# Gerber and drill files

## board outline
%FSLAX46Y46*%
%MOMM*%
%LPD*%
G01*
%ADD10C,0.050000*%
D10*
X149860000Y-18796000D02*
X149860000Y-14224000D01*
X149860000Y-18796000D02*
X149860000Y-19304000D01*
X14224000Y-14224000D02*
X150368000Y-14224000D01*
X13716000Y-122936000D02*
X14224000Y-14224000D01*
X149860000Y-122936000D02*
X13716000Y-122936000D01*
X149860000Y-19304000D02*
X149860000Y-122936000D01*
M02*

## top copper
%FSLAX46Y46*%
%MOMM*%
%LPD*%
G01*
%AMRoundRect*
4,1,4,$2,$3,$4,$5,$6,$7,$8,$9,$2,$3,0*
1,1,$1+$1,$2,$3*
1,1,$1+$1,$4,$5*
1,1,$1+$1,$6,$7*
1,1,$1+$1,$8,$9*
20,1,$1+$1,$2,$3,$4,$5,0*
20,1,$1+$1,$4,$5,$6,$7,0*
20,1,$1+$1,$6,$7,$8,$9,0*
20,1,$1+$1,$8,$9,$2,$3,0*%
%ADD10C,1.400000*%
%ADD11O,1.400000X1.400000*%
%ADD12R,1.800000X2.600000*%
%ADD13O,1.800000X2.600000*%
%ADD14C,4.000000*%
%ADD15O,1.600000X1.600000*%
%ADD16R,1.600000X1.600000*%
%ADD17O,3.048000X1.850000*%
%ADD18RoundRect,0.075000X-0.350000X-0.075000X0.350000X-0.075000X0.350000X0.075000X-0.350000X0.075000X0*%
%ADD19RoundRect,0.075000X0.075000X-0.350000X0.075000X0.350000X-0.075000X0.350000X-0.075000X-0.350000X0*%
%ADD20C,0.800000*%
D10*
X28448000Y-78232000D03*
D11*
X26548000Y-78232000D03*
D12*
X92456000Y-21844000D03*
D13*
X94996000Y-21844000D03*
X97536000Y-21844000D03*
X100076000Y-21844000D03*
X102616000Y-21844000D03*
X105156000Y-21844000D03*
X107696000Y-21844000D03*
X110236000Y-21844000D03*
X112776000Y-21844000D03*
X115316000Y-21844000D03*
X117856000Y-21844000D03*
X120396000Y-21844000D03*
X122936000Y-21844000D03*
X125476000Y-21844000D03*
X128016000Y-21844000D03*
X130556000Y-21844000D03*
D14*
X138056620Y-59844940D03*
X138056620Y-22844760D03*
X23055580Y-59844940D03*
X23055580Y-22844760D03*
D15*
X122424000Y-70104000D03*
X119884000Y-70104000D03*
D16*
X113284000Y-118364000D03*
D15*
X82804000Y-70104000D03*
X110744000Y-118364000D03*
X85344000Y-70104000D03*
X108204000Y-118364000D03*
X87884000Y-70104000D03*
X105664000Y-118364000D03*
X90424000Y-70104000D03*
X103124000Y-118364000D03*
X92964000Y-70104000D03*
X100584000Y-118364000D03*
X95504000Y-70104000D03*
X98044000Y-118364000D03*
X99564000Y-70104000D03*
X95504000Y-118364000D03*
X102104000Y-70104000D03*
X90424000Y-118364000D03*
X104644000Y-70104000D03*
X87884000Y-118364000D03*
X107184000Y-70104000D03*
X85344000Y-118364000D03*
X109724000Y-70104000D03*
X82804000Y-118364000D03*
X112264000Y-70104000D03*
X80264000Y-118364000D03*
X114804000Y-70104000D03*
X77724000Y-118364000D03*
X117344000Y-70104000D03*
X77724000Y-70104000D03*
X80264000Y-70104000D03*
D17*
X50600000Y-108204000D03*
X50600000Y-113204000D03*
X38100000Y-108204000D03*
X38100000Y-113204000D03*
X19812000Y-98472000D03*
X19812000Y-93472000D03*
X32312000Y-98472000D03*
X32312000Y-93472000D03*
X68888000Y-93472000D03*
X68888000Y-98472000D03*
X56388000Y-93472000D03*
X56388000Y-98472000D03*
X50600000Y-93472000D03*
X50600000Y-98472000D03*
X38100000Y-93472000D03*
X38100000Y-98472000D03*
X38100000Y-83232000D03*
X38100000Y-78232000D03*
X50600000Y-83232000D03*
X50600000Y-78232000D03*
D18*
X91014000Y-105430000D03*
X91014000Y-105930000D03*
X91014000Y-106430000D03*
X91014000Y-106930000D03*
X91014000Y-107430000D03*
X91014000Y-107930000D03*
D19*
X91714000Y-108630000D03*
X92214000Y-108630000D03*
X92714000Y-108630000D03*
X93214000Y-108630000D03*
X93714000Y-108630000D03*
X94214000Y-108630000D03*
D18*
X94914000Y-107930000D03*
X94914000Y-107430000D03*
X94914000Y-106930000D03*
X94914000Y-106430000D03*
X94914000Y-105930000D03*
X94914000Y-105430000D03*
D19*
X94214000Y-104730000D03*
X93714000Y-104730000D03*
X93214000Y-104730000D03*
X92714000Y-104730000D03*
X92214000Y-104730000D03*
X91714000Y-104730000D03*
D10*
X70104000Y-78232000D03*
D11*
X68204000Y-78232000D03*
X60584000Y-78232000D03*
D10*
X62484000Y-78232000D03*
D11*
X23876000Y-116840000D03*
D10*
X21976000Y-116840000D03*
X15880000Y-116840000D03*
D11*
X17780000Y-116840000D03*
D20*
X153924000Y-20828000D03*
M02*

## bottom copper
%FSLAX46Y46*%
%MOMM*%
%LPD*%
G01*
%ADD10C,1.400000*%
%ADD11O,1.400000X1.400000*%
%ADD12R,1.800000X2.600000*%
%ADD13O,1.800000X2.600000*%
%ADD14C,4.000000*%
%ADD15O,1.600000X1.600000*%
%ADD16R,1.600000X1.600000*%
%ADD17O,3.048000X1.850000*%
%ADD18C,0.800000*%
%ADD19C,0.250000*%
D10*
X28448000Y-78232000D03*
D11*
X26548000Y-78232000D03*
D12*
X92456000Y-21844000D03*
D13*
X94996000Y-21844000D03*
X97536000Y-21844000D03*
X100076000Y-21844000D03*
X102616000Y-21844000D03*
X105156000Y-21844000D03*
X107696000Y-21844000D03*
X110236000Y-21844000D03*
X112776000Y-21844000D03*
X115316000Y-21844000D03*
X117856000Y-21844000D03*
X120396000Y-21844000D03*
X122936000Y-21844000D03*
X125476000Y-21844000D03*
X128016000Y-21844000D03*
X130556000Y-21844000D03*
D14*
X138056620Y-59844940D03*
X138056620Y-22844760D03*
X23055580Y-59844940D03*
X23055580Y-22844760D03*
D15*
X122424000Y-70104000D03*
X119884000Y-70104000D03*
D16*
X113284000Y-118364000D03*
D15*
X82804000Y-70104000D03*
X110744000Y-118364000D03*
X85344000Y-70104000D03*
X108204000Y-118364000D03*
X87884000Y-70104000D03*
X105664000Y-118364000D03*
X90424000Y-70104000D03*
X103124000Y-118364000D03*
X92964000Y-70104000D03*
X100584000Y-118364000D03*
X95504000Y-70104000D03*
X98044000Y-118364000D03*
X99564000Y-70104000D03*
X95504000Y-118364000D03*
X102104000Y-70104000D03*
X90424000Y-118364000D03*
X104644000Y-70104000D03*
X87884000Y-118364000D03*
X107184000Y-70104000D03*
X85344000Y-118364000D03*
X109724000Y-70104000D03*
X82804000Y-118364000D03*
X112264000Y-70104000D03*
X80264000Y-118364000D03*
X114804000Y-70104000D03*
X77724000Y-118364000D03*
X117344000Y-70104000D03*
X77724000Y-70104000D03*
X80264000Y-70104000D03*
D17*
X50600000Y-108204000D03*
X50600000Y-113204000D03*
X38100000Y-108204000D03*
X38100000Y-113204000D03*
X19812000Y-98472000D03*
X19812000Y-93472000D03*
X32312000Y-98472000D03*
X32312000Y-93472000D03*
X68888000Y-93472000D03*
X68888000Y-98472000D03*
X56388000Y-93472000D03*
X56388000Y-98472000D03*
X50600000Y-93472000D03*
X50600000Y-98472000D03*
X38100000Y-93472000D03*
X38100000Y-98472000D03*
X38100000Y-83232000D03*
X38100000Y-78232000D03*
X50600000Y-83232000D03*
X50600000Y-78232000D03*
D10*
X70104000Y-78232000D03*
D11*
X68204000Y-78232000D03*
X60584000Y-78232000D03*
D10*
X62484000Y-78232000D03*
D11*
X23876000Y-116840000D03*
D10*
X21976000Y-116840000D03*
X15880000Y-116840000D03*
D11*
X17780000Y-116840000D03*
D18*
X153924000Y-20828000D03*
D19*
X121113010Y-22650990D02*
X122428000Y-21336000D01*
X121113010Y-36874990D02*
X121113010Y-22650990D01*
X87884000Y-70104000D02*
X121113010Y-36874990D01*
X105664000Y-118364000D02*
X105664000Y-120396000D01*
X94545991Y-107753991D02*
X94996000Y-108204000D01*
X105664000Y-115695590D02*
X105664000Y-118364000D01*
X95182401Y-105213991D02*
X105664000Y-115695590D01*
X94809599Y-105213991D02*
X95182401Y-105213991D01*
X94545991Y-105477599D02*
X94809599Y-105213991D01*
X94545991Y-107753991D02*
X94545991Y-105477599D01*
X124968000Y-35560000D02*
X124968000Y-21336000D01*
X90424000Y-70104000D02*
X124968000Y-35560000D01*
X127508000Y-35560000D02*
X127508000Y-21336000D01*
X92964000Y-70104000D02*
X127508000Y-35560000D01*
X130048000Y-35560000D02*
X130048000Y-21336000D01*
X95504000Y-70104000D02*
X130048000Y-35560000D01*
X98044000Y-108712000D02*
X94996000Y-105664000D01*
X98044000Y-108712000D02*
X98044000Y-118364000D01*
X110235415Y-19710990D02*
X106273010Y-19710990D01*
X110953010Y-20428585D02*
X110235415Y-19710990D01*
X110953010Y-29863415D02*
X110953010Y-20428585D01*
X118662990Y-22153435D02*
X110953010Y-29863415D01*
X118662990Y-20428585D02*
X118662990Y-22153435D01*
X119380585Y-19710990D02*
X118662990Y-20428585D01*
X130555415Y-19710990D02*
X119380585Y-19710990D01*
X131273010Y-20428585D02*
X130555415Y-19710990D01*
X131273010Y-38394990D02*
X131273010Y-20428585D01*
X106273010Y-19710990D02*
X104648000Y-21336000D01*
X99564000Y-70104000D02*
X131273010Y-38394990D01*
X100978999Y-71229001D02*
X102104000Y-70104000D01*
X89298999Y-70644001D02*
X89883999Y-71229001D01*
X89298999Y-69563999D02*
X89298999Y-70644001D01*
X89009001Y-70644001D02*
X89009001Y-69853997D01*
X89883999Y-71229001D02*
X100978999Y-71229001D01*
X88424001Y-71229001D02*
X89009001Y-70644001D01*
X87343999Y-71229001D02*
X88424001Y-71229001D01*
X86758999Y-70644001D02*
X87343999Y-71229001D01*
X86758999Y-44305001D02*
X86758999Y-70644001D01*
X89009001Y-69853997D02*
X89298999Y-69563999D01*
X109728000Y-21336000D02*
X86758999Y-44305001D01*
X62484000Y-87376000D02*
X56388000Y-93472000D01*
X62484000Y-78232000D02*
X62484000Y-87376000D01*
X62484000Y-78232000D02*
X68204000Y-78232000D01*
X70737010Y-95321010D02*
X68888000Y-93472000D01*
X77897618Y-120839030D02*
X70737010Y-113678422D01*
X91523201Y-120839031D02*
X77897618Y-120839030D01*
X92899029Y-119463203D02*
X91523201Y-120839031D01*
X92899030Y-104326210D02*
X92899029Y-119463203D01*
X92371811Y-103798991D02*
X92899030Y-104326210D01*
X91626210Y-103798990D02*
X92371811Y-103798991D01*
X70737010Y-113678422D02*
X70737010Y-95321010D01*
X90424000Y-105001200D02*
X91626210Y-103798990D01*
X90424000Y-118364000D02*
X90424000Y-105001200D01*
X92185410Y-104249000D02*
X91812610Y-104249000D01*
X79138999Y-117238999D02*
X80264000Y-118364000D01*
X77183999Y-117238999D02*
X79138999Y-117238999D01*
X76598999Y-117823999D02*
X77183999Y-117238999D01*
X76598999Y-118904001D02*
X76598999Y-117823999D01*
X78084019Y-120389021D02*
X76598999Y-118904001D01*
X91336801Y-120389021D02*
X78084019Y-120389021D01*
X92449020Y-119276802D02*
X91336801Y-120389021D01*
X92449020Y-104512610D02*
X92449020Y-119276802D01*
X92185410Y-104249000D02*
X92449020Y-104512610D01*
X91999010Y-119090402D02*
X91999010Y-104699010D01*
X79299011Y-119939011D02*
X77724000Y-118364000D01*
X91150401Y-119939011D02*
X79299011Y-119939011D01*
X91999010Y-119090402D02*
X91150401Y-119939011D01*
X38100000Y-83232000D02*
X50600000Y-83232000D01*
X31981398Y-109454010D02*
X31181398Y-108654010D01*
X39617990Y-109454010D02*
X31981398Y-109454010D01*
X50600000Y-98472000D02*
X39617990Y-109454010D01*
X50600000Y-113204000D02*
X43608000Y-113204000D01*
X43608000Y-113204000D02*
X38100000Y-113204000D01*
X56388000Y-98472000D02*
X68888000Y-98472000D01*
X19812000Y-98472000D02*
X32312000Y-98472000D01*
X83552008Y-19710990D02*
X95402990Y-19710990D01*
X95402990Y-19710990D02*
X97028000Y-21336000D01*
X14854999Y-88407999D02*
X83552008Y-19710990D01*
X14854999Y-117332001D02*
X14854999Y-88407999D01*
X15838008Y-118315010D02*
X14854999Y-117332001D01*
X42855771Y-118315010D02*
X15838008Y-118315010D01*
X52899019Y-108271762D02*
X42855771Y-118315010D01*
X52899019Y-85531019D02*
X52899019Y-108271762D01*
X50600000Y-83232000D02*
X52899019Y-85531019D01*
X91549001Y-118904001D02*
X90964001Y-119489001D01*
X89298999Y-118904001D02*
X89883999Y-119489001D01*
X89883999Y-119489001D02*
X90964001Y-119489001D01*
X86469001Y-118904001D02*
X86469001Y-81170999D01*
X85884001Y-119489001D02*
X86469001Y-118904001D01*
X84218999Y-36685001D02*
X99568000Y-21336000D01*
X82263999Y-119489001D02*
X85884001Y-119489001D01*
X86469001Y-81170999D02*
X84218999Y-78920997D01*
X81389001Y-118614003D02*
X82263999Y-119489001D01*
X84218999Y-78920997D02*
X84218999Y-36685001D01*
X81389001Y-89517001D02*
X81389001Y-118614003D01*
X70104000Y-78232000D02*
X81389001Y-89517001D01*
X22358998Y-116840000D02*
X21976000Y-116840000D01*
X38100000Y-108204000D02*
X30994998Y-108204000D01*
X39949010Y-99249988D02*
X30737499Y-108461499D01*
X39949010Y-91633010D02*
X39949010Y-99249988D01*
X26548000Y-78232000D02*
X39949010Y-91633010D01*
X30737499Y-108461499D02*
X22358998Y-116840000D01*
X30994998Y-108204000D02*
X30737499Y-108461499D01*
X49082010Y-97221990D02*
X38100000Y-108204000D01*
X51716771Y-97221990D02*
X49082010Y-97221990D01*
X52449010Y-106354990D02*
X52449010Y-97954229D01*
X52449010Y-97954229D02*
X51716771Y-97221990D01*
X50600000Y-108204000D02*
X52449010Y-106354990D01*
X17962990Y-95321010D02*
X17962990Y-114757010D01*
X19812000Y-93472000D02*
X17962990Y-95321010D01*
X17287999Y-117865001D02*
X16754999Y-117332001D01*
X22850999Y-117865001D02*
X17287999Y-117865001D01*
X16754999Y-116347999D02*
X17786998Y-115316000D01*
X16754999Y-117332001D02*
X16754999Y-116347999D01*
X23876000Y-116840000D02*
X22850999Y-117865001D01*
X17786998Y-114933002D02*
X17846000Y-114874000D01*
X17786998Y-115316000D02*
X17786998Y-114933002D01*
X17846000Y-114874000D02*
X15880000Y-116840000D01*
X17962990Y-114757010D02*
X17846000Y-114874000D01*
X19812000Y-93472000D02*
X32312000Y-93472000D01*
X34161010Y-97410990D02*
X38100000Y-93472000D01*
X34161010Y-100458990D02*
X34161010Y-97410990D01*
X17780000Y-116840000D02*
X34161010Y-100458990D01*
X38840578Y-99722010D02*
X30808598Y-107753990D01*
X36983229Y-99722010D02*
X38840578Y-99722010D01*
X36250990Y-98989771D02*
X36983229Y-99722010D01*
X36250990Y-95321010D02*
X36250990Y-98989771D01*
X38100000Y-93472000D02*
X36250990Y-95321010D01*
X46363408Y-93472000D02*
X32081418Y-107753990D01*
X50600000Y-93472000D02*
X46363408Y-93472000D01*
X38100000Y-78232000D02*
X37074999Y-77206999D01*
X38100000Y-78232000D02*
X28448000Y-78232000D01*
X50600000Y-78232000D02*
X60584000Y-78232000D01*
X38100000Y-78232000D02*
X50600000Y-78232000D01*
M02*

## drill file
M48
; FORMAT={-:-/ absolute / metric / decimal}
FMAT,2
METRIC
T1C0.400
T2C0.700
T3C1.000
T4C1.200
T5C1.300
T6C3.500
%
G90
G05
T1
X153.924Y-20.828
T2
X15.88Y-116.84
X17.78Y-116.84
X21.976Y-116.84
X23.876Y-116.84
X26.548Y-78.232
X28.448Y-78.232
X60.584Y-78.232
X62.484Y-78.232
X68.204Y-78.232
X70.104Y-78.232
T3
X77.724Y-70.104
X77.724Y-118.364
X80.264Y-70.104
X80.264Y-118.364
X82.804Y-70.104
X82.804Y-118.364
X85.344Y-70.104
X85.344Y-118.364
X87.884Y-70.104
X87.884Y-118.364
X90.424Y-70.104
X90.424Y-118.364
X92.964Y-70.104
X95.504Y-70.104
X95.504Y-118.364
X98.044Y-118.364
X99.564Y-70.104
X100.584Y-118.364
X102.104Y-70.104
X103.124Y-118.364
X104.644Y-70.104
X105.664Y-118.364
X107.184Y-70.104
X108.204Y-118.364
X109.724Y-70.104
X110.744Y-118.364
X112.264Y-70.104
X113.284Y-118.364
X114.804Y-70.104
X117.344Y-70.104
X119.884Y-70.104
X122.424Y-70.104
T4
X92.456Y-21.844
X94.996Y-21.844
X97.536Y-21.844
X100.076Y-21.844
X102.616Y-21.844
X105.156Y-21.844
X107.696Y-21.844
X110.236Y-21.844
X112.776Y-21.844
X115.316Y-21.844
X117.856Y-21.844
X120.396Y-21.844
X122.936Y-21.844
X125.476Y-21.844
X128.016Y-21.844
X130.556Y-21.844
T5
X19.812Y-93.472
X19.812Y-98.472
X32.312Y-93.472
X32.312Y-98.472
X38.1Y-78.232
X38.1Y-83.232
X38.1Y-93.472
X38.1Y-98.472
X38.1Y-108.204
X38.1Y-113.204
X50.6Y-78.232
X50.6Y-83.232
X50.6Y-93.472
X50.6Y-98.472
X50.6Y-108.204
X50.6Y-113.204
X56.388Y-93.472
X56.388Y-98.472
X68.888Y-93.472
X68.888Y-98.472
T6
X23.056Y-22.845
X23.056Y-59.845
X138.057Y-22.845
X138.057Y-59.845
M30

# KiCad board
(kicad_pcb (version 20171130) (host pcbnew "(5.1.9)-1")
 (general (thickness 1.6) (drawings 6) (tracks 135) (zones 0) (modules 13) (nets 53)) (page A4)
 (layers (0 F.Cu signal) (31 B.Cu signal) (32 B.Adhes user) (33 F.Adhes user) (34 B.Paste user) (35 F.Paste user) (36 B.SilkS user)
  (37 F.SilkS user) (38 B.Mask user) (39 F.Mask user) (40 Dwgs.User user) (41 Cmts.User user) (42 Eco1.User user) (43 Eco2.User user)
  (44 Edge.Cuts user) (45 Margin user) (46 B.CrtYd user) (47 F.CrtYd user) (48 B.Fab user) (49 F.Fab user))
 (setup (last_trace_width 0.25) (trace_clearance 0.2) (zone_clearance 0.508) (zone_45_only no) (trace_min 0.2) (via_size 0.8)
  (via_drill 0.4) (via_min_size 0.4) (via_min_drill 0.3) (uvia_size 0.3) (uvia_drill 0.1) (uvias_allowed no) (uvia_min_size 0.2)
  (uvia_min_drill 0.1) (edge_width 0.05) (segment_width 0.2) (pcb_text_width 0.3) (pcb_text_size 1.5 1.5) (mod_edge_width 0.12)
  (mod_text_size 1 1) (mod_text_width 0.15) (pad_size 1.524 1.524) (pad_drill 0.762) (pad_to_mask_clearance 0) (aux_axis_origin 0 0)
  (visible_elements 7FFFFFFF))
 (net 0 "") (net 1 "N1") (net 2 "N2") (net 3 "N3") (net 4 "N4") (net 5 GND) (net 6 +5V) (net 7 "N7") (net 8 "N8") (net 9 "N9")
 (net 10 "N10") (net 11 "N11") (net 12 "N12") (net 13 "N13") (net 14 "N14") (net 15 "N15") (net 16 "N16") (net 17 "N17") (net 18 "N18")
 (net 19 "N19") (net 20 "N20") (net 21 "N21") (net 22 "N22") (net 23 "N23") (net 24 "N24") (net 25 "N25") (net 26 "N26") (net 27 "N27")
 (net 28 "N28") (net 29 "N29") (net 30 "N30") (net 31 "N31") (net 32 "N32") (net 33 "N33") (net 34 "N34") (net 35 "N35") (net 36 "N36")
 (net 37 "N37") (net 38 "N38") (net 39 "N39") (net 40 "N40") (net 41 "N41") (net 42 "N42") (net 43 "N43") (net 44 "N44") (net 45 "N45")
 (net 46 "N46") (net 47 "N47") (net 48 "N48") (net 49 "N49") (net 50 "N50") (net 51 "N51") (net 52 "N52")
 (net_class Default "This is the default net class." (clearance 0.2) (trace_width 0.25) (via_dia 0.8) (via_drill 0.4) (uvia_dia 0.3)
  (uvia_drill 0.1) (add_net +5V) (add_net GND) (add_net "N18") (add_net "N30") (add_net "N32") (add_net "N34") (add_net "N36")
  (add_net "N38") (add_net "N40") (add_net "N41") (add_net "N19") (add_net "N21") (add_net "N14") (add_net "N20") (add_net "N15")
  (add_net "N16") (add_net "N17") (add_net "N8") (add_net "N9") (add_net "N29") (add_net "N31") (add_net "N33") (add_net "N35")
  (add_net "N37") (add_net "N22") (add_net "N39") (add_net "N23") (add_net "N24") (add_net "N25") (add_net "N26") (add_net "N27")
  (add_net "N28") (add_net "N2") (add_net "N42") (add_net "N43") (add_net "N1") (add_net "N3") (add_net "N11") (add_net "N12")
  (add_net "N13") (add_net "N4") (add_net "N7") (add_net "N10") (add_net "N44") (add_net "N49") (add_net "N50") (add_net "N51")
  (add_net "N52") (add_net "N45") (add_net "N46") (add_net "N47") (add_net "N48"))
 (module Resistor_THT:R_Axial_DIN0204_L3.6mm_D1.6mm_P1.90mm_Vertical (layer F.Cu) (at 28.448 78.232 180)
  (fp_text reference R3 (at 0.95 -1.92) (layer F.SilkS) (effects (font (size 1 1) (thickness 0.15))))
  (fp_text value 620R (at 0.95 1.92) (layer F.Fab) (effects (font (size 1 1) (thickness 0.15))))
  (pad 1 thru_hole circle (at 0 0 180) (size 1.4 1.4) (drill 0.7) (layers *.Cu *.Mask) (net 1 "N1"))
  (pad 2 thru_hole oval (at 1.9 0 180) (size 1.4 1.4) (drill 0.7) (layers *.Cu *.Mask) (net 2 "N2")))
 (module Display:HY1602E (layer F.Cu) (at 92.456 21.844)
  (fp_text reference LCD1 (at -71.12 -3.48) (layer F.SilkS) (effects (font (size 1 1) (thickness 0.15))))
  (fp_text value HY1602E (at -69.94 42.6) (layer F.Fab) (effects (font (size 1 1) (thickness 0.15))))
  (pad 1 thru_hole rect (at 0 0 180) (size 1.8 2.6) (drill 1.2) (layers *.Cu *.Mask) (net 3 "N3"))
  (pad 2 thru_hole oval (at 2.54 0 180) (size 1.8 2.6) (drill 1.2) (layers *.Cu *.Mask) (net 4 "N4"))
  (pad 3 thru_hole oval (at 5.08 0 180) (size 1.8 2.6) (drill 1.2) (layers *.Cu *.Mask) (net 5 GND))
  (pad 4 thru_hole oval (at 7.62 0 180) (size 1.8 2.6) (drill 1.2) (layers *.Cu *.Mask) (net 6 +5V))
  (pad 5 thru_hole oval (at 10.16 0 180) (size 1.8 2.6) (drill 1.2) (layers *.Cu *.Mask) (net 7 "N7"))
  (pad 6 thru_hole oval (at 12.7 0 180) (size 1.8 2.6) (drill 1.2) (layers *.Cu *.Mask) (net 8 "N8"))
  (pad 7 thru_hole oval (at 15.24 0 180) (size 1.8 2.6) (drill 1.2) (layers *.Cu *.Mask) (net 5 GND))
  (pad 8 thru_hole oval (at 17.78 0 180) (size 1.8 2.6) (drill 1.2) (layers *.Cu *.Mask) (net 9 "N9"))
  (pad 9 thru_hole oval (at 20.32 0 180) (size 1.8 2.6) (drill 1.2) (layers *.Cu *.Mask) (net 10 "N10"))
  (pad 10 thru_hole oval (at 22.86 0 180) (size 1.8 2.6) (drill 1.2) (layers *.Cu *.Mask) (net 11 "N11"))
  (pad 11 thru_hole oval (at 25.4 0 180) (size 1.8 2.6) (drill 1.2) (layers *.Cu *.Mask) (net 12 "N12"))
  (pad 12 thru_hole oval (at 27.94 0 180) (size 1.8 2.6) (drill 1.2) (layers *.Cu *.Mask) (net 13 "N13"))
  (pad 13 thru_hole oval (at 30.48 0 180) (size 1.8 2.6) (drill 1.2) (layers *.Cu *.Mask) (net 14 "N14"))
  (pad 14 thru_hole oval (at 33.02 0 180) (size 1.8 2.6) (drill 1.2) (layers *.Cu *.Mask) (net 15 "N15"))
  (pad 15 thru_hole oval (at 35.56 0 180) (size 1.8 2.6) (drill 1.2) (layers *.Cu *.Mask) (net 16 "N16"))
  (pad 16 thru_hole oval (at 38.1 0 180) (size 1.8 2.6) (drill 1.2) (layers *.Cu *.Mask) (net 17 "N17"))
  (pad "" thru_hole circle (at 45.60062 38.00094 180) (size 4 4) (drill 3.5) (layers *.Cu *.Mask))
  (pad "" thru_hole circle (at 45.60062 1.00076 180) (size 4 4) (drill 3.5) (layers *.Cu *.Mask))
  (pad "" thru_hole circle (at -69.40042 38.00094 180) (size 4 4) (drill 3.5) (layers *.Cu *.Mask))
  (pad "" thru_hole circle (at -69.40042 1.00076 180) (size 4 4) (drill 3.5) (layers *.Cu *.Mask)))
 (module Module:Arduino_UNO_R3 (layer F.Cu) (at 113.284 118.364 180)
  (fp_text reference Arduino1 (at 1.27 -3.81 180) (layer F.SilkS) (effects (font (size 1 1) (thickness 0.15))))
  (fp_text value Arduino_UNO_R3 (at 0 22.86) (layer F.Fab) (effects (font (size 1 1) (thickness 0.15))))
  (pad 32 thru_hole oval (at -9.14 48.26 270) (size 1.6 1.6) (drill 1) (layers *.Cu *.Mask))
  (pad 31 thru_hole oval (at -6.6 48.26 270) (size 1.6 1.6) (drill 1) (layers *.Cu *.Mask))
  (pad 1 thru_hole rect (at 0 0 270) (size 1.6 1.6) (drill 1) (layers *.Cu *.Mask) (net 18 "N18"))
  (pad 17 thru_hole oval (at 30.48 48.26 270) (size 1.6 1.6) (drill 1) (layers *.Cu *.Mask) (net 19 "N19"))
  (pad 2 thru_hole oval (at 2.54 0 270) (size 1.6 1.6) (drill 1) (layers *.Cu *.Mask) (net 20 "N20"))
  (pad 18 thru_hole oval (at 27.94 48.26 270) (size 1.6 1.6) (drill 1) (layers *.Cu *.Mask) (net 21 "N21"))
  (pad 3 thru_hole oval (at 5.08 0 270) (size 1.6 1.6) (drill 1) (layers *.Cu *.Mask) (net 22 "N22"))
  (pad 19 thru_hole oval (at 25.4 48.26 270) (size 1.6 1.6) (drill 1) (layers *.Cu *.Mask) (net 14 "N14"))
  (pad 4 thru_hole oval (at 7.62 0 270) (size 1.6 1.6) (drill 1) (layers *.Cu *.Mask) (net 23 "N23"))
  (pad 20 thru_hole oval (at 22.86 48.26 270) (size 1.6 1.6) (drill 1) (layers *.Cu *.Mask) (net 15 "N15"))
  (pad 5 thru_hole oval (at 10.16 0 270) (size 1.6 1.6) (drill 1) (layers *.Cu *.Mask) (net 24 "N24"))
  (pad 21 thru_hole oval (at 20.32 48.26 270) (size 1.6 1.6) (drill 1) (layers *.Cu *.Mask) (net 16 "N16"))
  (pad 6 thru_hole oval (at 12.7 0 270) (size 1.6 1.6) (drill 1) (layers *.Cu *.Mask) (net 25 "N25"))
  (pad 22 thru_hole oval (at 17.78 48.26 270) (size 1.6 1.6) (drill 1) (layers *.Cu *.Mask) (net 17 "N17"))
  (pad 7 thru_hole oval (at 15.24 0 270) (size 1.6 1.6) (drill 1) (layers *.Cu *.Mask) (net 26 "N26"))
  (pad 23 thru_hole oval (at 13.72 48.26 270) (size 1.6 1.6) (drill 1) (layers *.Cu *.Mask) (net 8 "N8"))
  (pad 8 thru_hole oval (at 17.78 0 270) (size 1.6 1.6) (drill 1) (layers *.Cu *.Mask) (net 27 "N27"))
  (pad 24 thru_hole oval (at 11.18 48.26 270) (size 1.6 1.6) (drill 1) (layers *.Cu *.Mask) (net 9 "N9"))
  (pad 9 thru_hole oval (at 22.86 0 270) (size 1.6 1.6) (drill 1) (layers *.Cu *.Mask) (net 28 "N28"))
  (pad 25 thru_hole oval (at 8.64 48.26 270) (size 1.6 1.6) (drill 1) (layers *.Cu *.Mask) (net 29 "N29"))
  (pad 10 thru_hole oval (at 25.4 0 270) (size 1.6 1.6) (drill 1) (layers *.Cu *.Mask) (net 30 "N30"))
  (pad 26 thru_hole oval (at 6.1 48.26 270) (size 1.6 1.6) (drill 1) (layers *.Cu *.Mask) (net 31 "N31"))
  (pad 11 thru_hole oval (at 27.94 0 270) (size 1.6 1.6) (drill 1) (layers *.Cu *.Mask) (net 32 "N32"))
  (pad 27 thru_hole oval (at 3.56 48.26 270) (size 1.6 1.6) (drill 1) (layers *.Cu *.Mask) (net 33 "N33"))
  (pad 12 thru_hole oval (at 30.48 0 270) (size 1.6 1.6) (drill 1) (layers *.Cu *.Mask) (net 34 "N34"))
  (pad 28 thru_hole oval (at 1.02 48.26 270) (size 1.6 1.6) (drill 1) (layers *.Cu *.Mask) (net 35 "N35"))
  (pad 13 thru_hole oval (at 33.02 0 270) (size 1.6 1.6) (drill 1) (layers *.Cu *.Mask) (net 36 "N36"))
  (pad 29 thru_hole oval (at -1.52 48.26 270) (size 1.6 1.6) (drill 1) (layers *.Cu *.Mask) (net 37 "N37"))
  (pad 14 thru_hole oval (at 35.56 0 270) (size 1.6 1.6) (drill 1) (layers *.Cu *.Mask) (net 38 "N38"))
  (pad 30 thru_hole oval (at -4.06 48.26 270) (size 1.6 1.6) (drill 1) (layers *.Cu *.Mask) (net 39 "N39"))
  (pad 15 thru_hole oval (at 35.56 48.26 270) (size 1.6 1.6) (drill 1) (layers *.Cu *.Mask) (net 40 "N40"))
  (pad 16 thru_hole oval (at 33.02 48.26 270) (size 1.6 1.6) (drill 1) (layers *.Cu *.Mask) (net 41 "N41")))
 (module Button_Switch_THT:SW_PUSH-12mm (layer F.Cu) (at 38.1 108.204)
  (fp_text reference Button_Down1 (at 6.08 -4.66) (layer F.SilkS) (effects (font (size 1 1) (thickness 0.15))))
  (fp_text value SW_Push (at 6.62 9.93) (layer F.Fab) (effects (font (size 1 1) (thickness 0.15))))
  (pad 1 thru_hole oval (at 12.5 0) (size 3.048 1.85) (drill 1.3) (layers *.Cu *.Mask) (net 2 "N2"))
  (pad 2 thru_hole oval (at 12.5 5) (size 3.048 1.85) (drill 1.3) (layers *.Cu *.Mask) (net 5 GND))
  (pad 1 thru_hole oval (at 0 0) (size 3.048 1.85) (drill 1.3) (layers *.Cu *.Mask) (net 2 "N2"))
  (pad 2 thru_hole oval (at 0 5) (size 3.048 1.85) (drill 1.3) (layers *.Cu *.Mask) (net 5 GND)))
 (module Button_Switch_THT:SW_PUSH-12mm (layer F.Cu) (at 19.812 93.472)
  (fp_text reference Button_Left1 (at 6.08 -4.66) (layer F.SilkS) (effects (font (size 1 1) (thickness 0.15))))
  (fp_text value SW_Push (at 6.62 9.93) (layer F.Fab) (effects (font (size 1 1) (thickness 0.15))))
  (pad 2 thru_hole oval (at 0 5) (size 3.048 1.85) (drill 1.3) (layers *.Cu *.Mask) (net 5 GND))
  (pad 1 thru_hole oval (at 0 0) (size 3.048 1.85) (drill 1.3) (layers *.Cu *.Mask) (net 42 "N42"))
  (pad 2 thru_hole oval (at 12.5 5) (size 3.048 1.85) (drill 1.3) (layers *.Cu *.Mask) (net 5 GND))
  (pad 1 thru_hole oval (at 12.5 0) (size 3.048 1.85) (drill 1.3) (layers *.Cu *.Mask) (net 42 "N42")))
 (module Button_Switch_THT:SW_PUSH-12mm (layer F.Cu) (at 56.388 93.472)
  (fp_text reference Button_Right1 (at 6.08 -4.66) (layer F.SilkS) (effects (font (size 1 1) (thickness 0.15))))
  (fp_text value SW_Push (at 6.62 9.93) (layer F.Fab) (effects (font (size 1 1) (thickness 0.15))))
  (pad 1 thru_hole oval (at 12.5 0) (size 3.048 1.85) (drill 1.3) (layers *.Cu *.Mask) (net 28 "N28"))
  (pad 2 thru_hole oval (at 12.5 5) (size 3.048 1.85) (drill 1.3) (layers *.Cu *.Mask) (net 5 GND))
  (pad 1 thru_hole oval (at 0 0) (size 3.048 1.85) (drill 1.3) (layers *.Cu *.Mask) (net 28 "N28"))
  (pad 2 thru_hole oval (at 0 5) (size 3.048 1.85) (drill 1.3) (layers *.Cu *.Mask) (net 5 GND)))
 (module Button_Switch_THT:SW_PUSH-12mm (layer F.Cu) (at 38.1 93.472)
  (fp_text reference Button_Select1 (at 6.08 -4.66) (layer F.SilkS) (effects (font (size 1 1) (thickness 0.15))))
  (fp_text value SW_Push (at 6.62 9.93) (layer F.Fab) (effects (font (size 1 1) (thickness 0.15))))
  (pad 1 thru_hole oval (at 12.5 0) (size 3.048 1.85) (drill 1.3) (layers *.Cu *.Mask) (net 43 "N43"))
  (pad 2 thru_hole oval (at 12.5 5) (size 3.048 1.85) (drill 1.3) (layers *.Cu *.Mask) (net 5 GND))
  (pad 1 thru_hole oval (at 0 0) (size 3.048 1.85) (drill 1.3) (layers *.Cu *.Mask) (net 43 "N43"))
  (pad 2 thru_hole oval (at 0 5) (size 3.048 1.85) (drill 1.3) (layers *.Cu *.Mask) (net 5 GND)))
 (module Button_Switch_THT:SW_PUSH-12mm (layer F.Cu) (at 38.1 78.232)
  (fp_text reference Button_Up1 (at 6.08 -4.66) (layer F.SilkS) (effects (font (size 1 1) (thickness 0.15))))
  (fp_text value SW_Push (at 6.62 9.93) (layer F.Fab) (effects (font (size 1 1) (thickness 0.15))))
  (pad 2 thru_hole oval (at 0 5) (size 3.048 1.85) (drill 1.3) (layers *.Cu *.Mask) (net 5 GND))
  (pad 1 thru_hole oval (at 0 0) (size 3.048 1.85) (drill 1.3) (layers *.Cu *.Mask) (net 1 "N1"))
  (pad 2 thru_hole oval (at 12.5 5) (size 3.048 1.85) (drill 1.3) (layers *.Cu *.Mask) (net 5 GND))
  (pad 1 thru_hole oval (at 12.5 0) (size 3.048 1.85) (drill 1.3) (layers *.Cu *.Mask) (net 1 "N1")))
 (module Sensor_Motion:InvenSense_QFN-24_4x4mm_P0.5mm (layer F.Cu) (at 92.964 106.68)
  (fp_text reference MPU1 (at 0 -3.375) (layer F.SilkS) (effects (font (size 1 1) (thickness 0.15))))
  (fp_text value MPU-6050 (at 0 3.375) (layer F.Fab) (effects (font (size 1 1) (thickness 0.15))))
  (pad 1 smd roundrect (at -1.95 -1.25) (size 0.85 0.3) (layers F.Cu F.Paste F.Mask) (roundrect_rratio 0.25) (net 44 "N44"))
  (pad 2 smd roundrect (at -1.95 -0.75) (size 0.85 0.3) (layers F.Cu F.Paste F.Mask) (roundrect_rratio 0.25))
  (pad 3 smd roundrect (at -1.95 -0.25) (size 0.85 0.3) (layers F.Cu F.Paste F.Mask) (roundrect_rratio 0.25))
  (pad 4 smd roundrect (at -1.95 0.25) (size 0.85 0.3) (layers F.Cu F.Paste F.Mask) (roundrect_rratio 0.25))
  (pad 5 smd roundrect (at -1.95 0.75) (size 0.85 0.3) (layers F.Cu F.Paste F.Mask) (roundrect_rratio 0.25))
  (pad 6 smd roundrect (at -1.95 1.25) (size 0.85 0.3) (layers F.Cu F.Paste F.Mask) (roundrect_rratio 0.25) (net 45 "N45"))
  (pad 7 smd roundrect (at -1.25 1.95 90) (size 0.85 0.3) (layers F.Cu F.Paste F.Mask) (roundrect_rratio 0.25) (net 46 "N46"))
  (pad 8 smd roundrect (at -0.75 1.95 90) (size 0.85 0.3) (layers F.Cu F.Paste F.Mask) (roundrect_rratio 0.25) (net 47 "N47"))
  (pad 9 smd roundrect (at -0.25 1.95 90) (size 0.85 0.3) (layers F.Cu F.Paste F.Mask) (roundrect_rratio 0.25) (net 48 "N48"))
  (pad 10 smd roundrect (at 0.25 1.95 90) (size 0.85 0.3) (layers F.Cu F.Paste F.Mask) (roundrect_rratio 0.25) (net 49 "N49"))
  (pad 11 smd roundrect (at 0.75 1.95 90) (size 0.85 0.3) (layers F.Cu F.Paste F.Mask) (roundrect_rratio 0.25) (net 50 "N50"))
  (pad 12 smd roundrect (at 1.25 1.95 90) (size 0.85 0.3) (layers F.Cu F.Paste F.Mask) (roundrect_rratio 0.25) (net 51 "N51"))
  (pad 13 smd roundrect (at 1.95 1.25) (size 0.85 0.3) (layers F.Cu F.Paste F.Mask) (roundrect_rratio 0.25) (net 23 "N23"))
  (pad 14 smd roundrect (at 1.95 0.75) (size 0.85 0.3) (layers F.Cu F.Paste F.Mask) (roundrect_rratio 0.25))
  (pad 15 smd roundrect (at 1.95 0.25) (size 0.85 0.3) (layers F.Cu F.Paste F.Mask) (roundrect_rratio 0.25))
  (pad 16 smd roundrect (at 1.95 -0.25) (size 0.85 0.3) (layers F.Cu F.Paste F.Mask) (roundrect_rratio 0.25))
  (pad 17 smd roundrect (at 1.95 -0.75) (size 0.85 0.3) (layers F.Cu F.Paste F.Mask) (roundrect_rratio 0.25))
  (pad 18 smd roundrect (at 1.95 -1.25) (size 0.85 0.3) (layers F.Cu F.Paste F.Mask) (roundrect_rratio 0.25) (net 26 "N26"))
  (pad 19 smd roundrect (at 1.25 -1.95 90) (size 0.85 0.3) (layers F.Cu F.Paste F.Mask) (roundrect_rratio 0.25))
  (pad 20 smd roundrect (at 0.75 -1.95 90) (size 0.85 0.3) (layers F.Cu F.Paste F.Mask) (roundrect_rratio 0.25) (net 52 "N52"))
  (pad 21 smd roundrect (at 0.25 -1.95 90) (size 0.85 0.3) (layers F.Cu F.Paste F.Mask) (roundrect_rratio 0.25))
  (pad 22 smd roundrect (at -0.25 -1.95 90) (size 0.85 0.3) (layers F.Cu F.Paste F.Mask) (roundrect_rratio 0.25))
  (pad 23 smd roundrect (at -0.75 -1.95 90) (size 0.85 0.3) (layers F.Cu F.Paste F.Mask) (roundrect_rratio 0.25) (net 38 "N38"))
  (pad 24 smd roundrect (at -1.25 -1.95 90) (size 0.85 0.3) (layers F.Cu F.Paste F.Mask) (roundrect_rratio 0.25) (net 36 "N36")))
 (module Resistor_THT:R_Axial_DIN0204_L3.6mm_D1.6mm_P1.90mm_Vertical (layer F.Cu) (at 70.104 78.232 180)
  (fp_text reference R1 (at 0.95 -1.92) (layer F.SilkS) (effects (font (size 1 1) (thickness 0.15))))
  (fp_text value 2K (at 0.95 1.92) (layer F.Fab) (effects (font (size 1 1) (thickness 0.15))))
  (pad 1 thru_hole circle (at 0 0 180) (size 1.4 1.4) (drill 0.7) (layers *.Cu *.Mask) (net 6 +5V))
  (pad 2 thru_hole oval (at 1.9 0 180) (size 1.4 1.4) (drill 0.7) (layers *.Cu *.Mask) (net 28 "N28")))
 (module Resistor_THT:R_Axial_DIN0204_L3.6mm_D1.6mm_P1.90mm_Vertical (layer F.Cu) (at 62.484 78.232 180)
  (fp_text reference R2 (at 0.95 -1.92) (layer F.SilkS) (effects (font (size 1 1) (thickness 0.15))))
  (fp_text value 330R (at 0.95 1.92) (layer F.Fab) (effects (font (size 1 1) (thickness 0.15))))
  (pad 2 thru_hole oval (at 1.9 0 180) (size 1.4 1.4) (drill 0.7) (layers *.Cu *.Mask) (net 1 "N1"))
  (pad 1 thru_hole circle (at 0 0 180) (size 1.4 1.4) (drill 0.7) (layers *.Cu *.Mask) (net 28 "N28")))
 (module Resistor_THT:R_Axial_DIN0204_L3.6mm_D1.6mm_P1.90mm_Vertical (layer F.Cu) (at 21.976 116.84)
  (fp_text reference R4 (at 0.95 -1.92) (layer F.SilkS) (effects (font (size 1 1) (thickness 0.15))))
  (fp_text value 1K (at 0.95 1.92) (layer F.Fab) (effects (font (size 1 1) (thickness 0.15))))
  (pad 2 thru_hole oval (at 1.9 0) (size 1.4 1.4) (drill 0.7) (layers *.Cu *.Mask) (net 42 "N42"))
  (pad 1 thru_hole circle (at 0 0) (size 1.4 1.4) (drill 0.7) (layers *.Cu *.Mask) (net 2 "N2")))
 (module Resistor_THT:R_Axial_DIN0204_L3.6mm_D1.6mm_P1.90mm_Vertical (layer F.Cu) (at 15.88 116.84)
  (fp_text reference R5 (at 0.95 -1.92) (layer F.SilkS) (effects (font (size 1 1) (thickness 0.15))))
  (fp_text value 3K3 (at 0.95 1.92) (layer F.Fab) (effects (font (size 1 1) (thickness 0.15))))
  (pad 1 thru_hole circle (at 0 0) (size 1.4 1.4) (drill 0.7) (layers *.Cu *.Mask) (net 42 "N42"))
  (pad 2 thru_hole oval (at 1.9 0) (size 1.4 1.4) (drill 0.7) (layers *.Cu *.Mask) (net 43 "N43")))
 (gr_line (start 149.86 18.796) (end 149.86 14.224) (layer Edge.Cuts) (width 0.05))
 (gr_line (start 149.86 18.796) (end 149.86 19.304) (layer Edge.Cuts) (width 0.05))
 (gr_line (start 14.224 14.224) (end 150.368 14.224) (layer Edge.Cuts) (width 0.05))
 (gr_line (start 13.716 122.936) (end 14.224 14.224) (layer Edge.Cuts) (width 0.05))
 (gr_line (start 149.86 122.936) (end 13.716 122.936) (layer Edge.Cuts) (width 0.05))
 (gr_line (start 149.86 19.304) (end 149.86 122.936) (layer Edge.Cuts) (width 0.05))
 (via (at 153.924 20.828) (size 0.8) (drill 0.4) (layers F.Cu B.Cu) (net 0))
 (segment (start 121.11301 22.65099) (end 122.428 21.336) (width 0.25) (layer B.Cu) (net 14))
 (segment (start 121.11301 36.87499) (end 121.11301 22.65099) (width 0.25) (layer B.Cu) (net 14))
 (segment (start 87.884 70.104) (end 121.11301 36.87499) (width 0.25) (layer B.Cu) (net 14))
 (segment (start 105.664 118.364) (end 105.664 120.396) (width 0.25) (layer B.Cu) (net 23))
 (segment (start 94.545991 107.753991) (end 94.996 108.204) (width 0.25) (layer B.Cu) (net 23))
 (segment (start 105.664 115.69559) (end 105.664 118.364) (width 0.25) (layer B.Cu) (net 23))
 (segment (start 95.182401 105.213991) (end 105.664 115.69559) (width 0.25) (layer B.Cu) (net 23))
 (segment (start 94.809599 105.213991) (end 95.182401 105.213991) (width 0.25) (layer B.Cu) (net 23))
 (segment (start 94.545991 105.477599) (end 94.809599 105.213991) (width 0.25) (layer B.Cu) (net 23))
 (segment (start 94.545991 107.753991) (end 94.545991 105.477599) (width 0.25) (layer B.Cu) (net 23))
 (segment (start 124.968 35.56) (end 124.968 21.336) (width 0.25) (layer B.Cu) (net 15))
 (segment (start 90.424 70.104) (end 124.968 35.56) (width 0.25) (layer B.Cu) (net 15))
 (segment (start 127.508 35.56) (end 127.508 21.336) (width 0.25) (layer B.Cu) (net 16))
 (segment (start 92.964 70.104) (end 127.508 35.56) (width 0.25) (layer B.Cu) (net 16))
 (segment (start 130.048 35.56) (end 130.048 21.336) (width 0.25) (layer B.Cu) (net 17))
 (segment (start 95.504 70.104) (end 130.048 35.56) (width 0.25) (layer B.Cu) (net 17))
 (segment (start 98.044 108.712) (end 94.996 105.664) (width 0.25) (layer B.Cu) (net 26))
 (segment (start 98.044 108.712) (end 98.044 118.364) (width 0.25) (layer B.Cu) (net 26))
 (segment (start 110.235415 19.71099) (end 106.27301 19.71099) (width 0.25) (layer B.Cu) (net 8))
 (segment (start 110.95301 20.428585) (end 110.235415 19.71099) (width 0.25) (layer B.Cu) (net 8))
 (segment (start 110.95301 29.863415) (end 110.95301 20.428585) (width 0.25) (layer B.Cu) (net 8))
 (segment (start 118.66299 22.153435) (end 110.95301 29.863415) (width 0.25) (layer B.Cu) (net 8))
 (segment (start 118.66299 20.428585) (end 118.66299 22.153435) (width 0.25) (layer B.Cu) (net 8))
 (segment (start 119.380585 19.71099) (end 118.66299 20.428585) (width 0.25) (layer B.Cu) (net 8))
 (segment (start 130.555415 19.71099) (end 119.380585 19.71099) (width 0.25) (layer B.Cu) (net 8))
 (segment (start 131.27301 20.428585) (end 130.555415 19.71099) (width 0.25) (layer B.Cu) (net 8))
 (segment (start 131.27301 38.39499) (end 131.27301 20.428585) (width 0.25) (layer B.Cu) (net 8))
 (segment (start 106.27301 19.71099) (end 104.648 21.336) (width 0.25) (layer B.Cu) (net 8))
 (segment (start 99.564 70.104) (end 131.27301 38.39499) (width 0.25) (layer B.Cu) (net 8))
 (segment (start 100.978999 71.229001) (end 102.104 70.104) (width 0.25) (layer B.Cu) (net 9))
 (segment (start 89.298999 70.644001) (end 89.883999 71.229001) (width 0.25) (layer B.Cu) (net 9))
 (segment (start 89.298999 69.563999) (end 89.298999 70.644001) (width 0.25) (layer B.Cu) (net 9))
 (segment (start 89.009001 70.644001) (end 89.009001 69.853997) (width 0.25) (layer B.Cu) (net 9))
 (segment (start 89.883999 71.229001) (end 100.978999 71.229001) (width 0.25) (layer B.Cu) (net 9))
 (segment (start 88.424001 71.229001) (end 89.009001 70.644001) (width 0.25) (layer B.Cu) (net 9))
 (segment (start 87.343999 71.229001) (end 88.424001 71.229001) (width 0.25) (layer B.Cu) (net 9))
 (segment (start 86.758999 70.644001) (end 87.343999 71.229001) (width 0.25) (layer B.Cu) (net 9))
 (segment (start 86.758999 44.305001) (end 86.758999 70.644001) (width 0.25) (layer B.Cu) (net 9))
 (segment (start 89.009001 69.853997) (end 89.298999 69.563999) (width 0.25) (layer B.Cu) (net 9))
 (segment (start 109.728 21.336) (end 86.758999 44.305001) (width 0.25) (layer B.Cu) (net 9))
 (segment (start 62.484 87.376) (end 56.388 93.472) (width 0.25) (layer B.Cu) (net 28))
 (segment (start 62.484 78.232) (end 62.484 87.376) (width 0.25) (layer B.Cu) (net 28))
 (segment (start 62.484 78.232) (end 68.204 78.232) (width 0.25) (layer B.Cu) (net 28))
 (segment (start 70.73701 95.32101) (end 68.888 93.472) (width 0.25) (layer B.Cu) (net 28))
 (segment (start 77.897618 120.83903) (end 70.73701 113.678422) (width 0.25) (layer B.Cu) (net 28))
 (segment (start 91.523201 120.839031) (end 77.897618 120.83903) (width 0.25) (layer B.Cu) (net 28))
 (segment (start 92.899029 119.463203) (end 91.523201 120.839031) (width 0.25) (layer B.Cu) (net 28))
 (segment (start 92.89903 104.32621) (end 92.899029 119.463203) (width 0.25) (layer B.Cu) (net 28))
 (segment (start 92.371811 103.798991) (end 92.89903 104.32621) (width 0.25) (layer B.Cu) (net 28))
 (segment (start 91.62621 103.79899) (end 92.371811 103.798991) (width 0.25) (layer B.Cu) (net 28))
 (segment (start 70.73701 113.678422) (end 70.73701 95.32101) (width 0.25) (layer B.Cu) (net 28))
 (segment (start 90.424 105.0012) (end 91.62621 103.79899) (width 0.25) (layer B.Cu) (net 28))
 (segment (start 90.424 118.364) (end 90.424 105.0012) (width 0.25) (layer B.Cu) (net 28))
 (segment (start 92.18541 104.249) (end 91.81261 104.249) (width 0.25) (layer B.Cu) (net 36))
 (segment (start 79.138999 117.238999) (end 80.264 118.364) (width 0.25) (layer B.Cu) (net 36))
 (segment (start 77.183999 117.238999) (end 79.138999 117.238999) (width 0.25) (layer B.Cu) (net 36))
 (segment (start 76.598999 117.823999) (end 77.183999 117.238999) (width 0.25) (layer B.Cu) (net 36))
 (segment (start 76.598999 118.904001) (end 76.598999 117.823999) (width 0.25) (layer B.Cu) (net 36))
 (segment (start 78.084019 120.389021) (end 76.598999 118.904001) (width 0.25) (layer B.Cu) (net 36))
 (segment (start 91.336801 120.389021) (end 78.084019 120.389021) (width 0.25) (layer B.Cu) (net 36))
 (segment (start 92.44902 119.276802) (end 91.336801 120.389021) (width 0.25) (layer B.Cu) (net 36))
 (segment (start 92.44902 104.51261) (end 92.44902 119.276802) (width 0.25) (layer B.Cu) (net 36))
 (segment (start 92.18541 104.249) (end 92.44902 104.51261) (width 0.25) (layer B.Cu) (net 36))
 (segment (start 91.99901 119.090402) (end 91.99901 104.69901) (width 0.25) (layer B.Cu) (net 38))
 (segment (start 79.299011 119.939011) (end 77.724 118.364) (width 0.25) (layer B.Cu) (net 38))
 (segment (start 91.150401 119.939011) (end 79.299011 119.939011) (width 0.25) (layer B.Cu) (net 38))
 (segment (start 91.99901 119.090402) (end 91.150401 119.939011) (width 0.25) (layer B.Cu) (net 38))
 (segment (start 38.1 83.232) (end 50.6 83.232) (width 0.25) (layer B.Cu) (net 5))
 (segment (start 31.981398 109.45401) (end 31.181398 108.65401) (width 0.25) (layer B.Cu) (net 5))
 (segment (start 39.61799 109.45401) (end 31.981398 109.45401) (width 0.25) (layer B.Cu) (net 5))
 (segment (start 50.6 98.472) (end 39.61799 109.45401) (width 0.25) (layer B.Cu) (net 5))
 (segment (start 50.6 113.204) (end 43.608 113.204) (width 0.25) (layer B.Cu) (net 5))
 (segment (start 43.608 113.204) (end 38.1 113.204) (width 0.25) (layer B.Cu) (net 5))
 (segment (start 56.388 98.472) (end 68.888 98.472) (width 0.25) (layer B.Cu) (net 5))
 (segment (start 19.812 98.472) (end 32.312 98.472) (width 0.25) (layer B.Cu) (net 5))
 (segment (start 83.552008 19.71099) (end 95.40299 19.71099) (width 0.25) (layer B.Cu) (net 5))
 (segment (start 95.40299 19.71099) (end 97.028 21.336) (width 0.25) (layer B.Cu) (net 5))
 (segment (start 14.854999 88.407999) (end 83.552008 19.71099) (width 0.25) (layer B.Cu) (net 5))
 (segment (start 14.854999 117.332001) (end 14.854999 88.407999) (width 0.25) (layer B.Cu) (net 5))
 (segment (start 15.838008 118.31501) (end 14.854999 117.332001) (width 0.25) (layer B.Cu) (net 5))
 (segment (start 42.855771 118.31501) (end 15.838008 118.31501) (width 0.25) (layer B.Cu) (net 5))
 (segment (start 52.899019 108.271762) (end 42.855771 118.31501) (width 0.25) (layer B.Cu) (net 5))
 (segment (start 52.899019 85.531019) (end 52.899019 108.271762) (width 0.25) (layer B.Cu) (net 5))
 (segment (start 50.6 83.232) (end 52.899019 85.531019) (width 0.25) (layer B.Cu) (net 5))
 (segment (start 91.549001 118.904001) (end 90.964001 119.489001) (width 0.25) (layer B.Cu) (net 6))
 (segment (start 89.298999 118.904001) (end 89.883999 119.489001) (width 0.25) (layer B.Cu) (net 6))
 (segment (start 89.883999 119.489001) (end 90.964001 119.489001) (width 0.25) (layer B.Cu) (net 6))
 (segment (start 86.469001 118.904001) (end 86.469001 81.170999) (width 0.25) (layer B.Cu) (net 6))
 (segment (start 85.884001 119.489001) (end 86.469001 118.904001) (width 0.25) (layer B.Cu) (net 6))
 (segment (start 84.218999 36.685001) (end 99.568 21.336) (width 0.25) (layer B.Cu) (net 6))
 (segment (start 82.263999 119.489001) (end 85.884001 119.489001) (width 0.25) (layer B.Cu) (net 6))
 (segment (start 86.469001 81.170999) (end 84.218999 78.920997) (width 0.25) (layer B.Cu) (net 6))
 (segment (start 81.389001 118.614003) (end 82.263999 119.489001) (width 0.25) (layer B.Cu) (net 6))
 (segment (start 84.218999 78.920997) (end 84.218999 36.685001) (width 0.25) (layer B.Cu) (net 6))
 (segment (start 81.389001 89.517001) (end 81.389001 118.614003) (width 0.25) (layer B.Cu) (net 6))
 (segment (start 70.104 78.232) (end 81.389001 89.517001) (width 0.25) (layer B.Cu) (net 6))
 (segment (start 22.358998 116.84) (end 21.976 116.84) (width 0.25) (layer B.Cu) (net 2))
 (segment (start 38.1 108.204) (end 30.994998 108.204) (width 0.25) (layer B.Cu) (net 2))
 (segment (start 39.94901 99.249988) (end 30.737499 108.461499) (width 0.25) (layer B.Cu) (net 2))
 (segment (start 39.94901 91.63301) (end 39.94901 99.249988) (width 0.25) (layer B.Cu) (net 2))
 (segment (start 26.548 78.232) (end 39.94901 91.63301) (width 0.25) (layer B.Cu) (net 2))
 (segment (start 30.737499 108.461499) (end 22.358998 116.84) (width 0.25) (layer B.Cu) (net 2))
 (segment (start 30.994998 108.204) (end 30.737499 108.461499) (width 0.25) (layer B.Cu) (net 2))
 (segment (start 49.08201 97.22199) (end 38.1 108.204) (width 0.25) (layer B.Cu) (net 2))
 (segment (start 51.716771 97.22199) (end 49.08201 97.22199) (width 0.25) (layer B.Cu) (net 2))
 (segment (start 52.44901 106.35499) (end 52.44901 97.954229) (width 0.25) (layer B.Cu) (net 2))
 (segment (start 52.44901 97.954229) (end 51.716771 97.22199) (width 0.25) (layer B.Cu) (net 2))
 (segment (start 50.6 108.204) (end 52.44901 106.35499) (width 0.25) (layer B.Cu) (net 2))
 (segment (start 17.96299 95.32101) (end 17.96299 114.75701) (width 0.25) (layer B.Cu) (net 42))
 (segment (start 19.812 93.472) (end 17.96299 95.32101) (width 0.25) (layer B.Cu) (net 42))
 (segment (start 17.287999 117.865001) (end 16.754999 117.332001) (width 0.25) (layer B.Cu) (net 42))
 (segment (start 22.850999 117.865001) (end 17.287999 117.865001) (width 0.25) (layer B.Cu) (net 42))
 (segment (start 16.754999 116.347999) (end 17.786998 115.316) (width 0.25) (layer B.Cu) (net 42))
 (segment (start 16.754999 117.332001) (end 16.754999 116.347999) (width 0.25) (layer B.Cu) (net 42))
 (segment (start 23.876 116.84) (end 22.850999 117.865001) (width 0.25) (layer B.Cu) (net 42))
 (segment (start 17.786998 114.933002) (end 17.846 114.874) (width 0.25) (layer B.Cu) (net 42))
 (segment (start 17.786998 115.316) (end 17.786998 114.933002) (width 0.25) (layer B.Cu) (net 42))
 (segment (start 17.846 114.874) (end 15.88 116.84) (width 0.25) (layer B.Cu) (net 42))
 (segment (start 17.96299 114.75701) (end 17.846 114.874) (width 0.25) (layer B.Cu) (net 42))
 (segment (start 19.812 93.472) (end 32.312 93.472) (width 0.25) (layer B.Cu) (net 42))
 (segment (start 34.16101 97.41099) (end 38.1 93.472) (width 0.25) (layer B.Cu) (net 43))
 (segment (start 34.16101 100.45899) (end 34.16101 97.41099) (width 0.25) (layer B.Cu) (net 43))
 (segment (start 17.78 116.84) (end 34.16101 100.45899) (width 0.25) (layer B.Cu) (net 43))
 (segment (start 38.840578 99.72201) (end 30.808598 107.75399) (width 0.25) (layer B.Cu) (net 43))
 (segment (start 36.983229 99.72201) (end 38.840578 99.72201) (width 0.25) (layer B.Cu) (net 43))
 (segment (start 36.25099 98.989771) (end 36.983229 99.72201) (width 0.25) (layer B.Cu) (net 43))
 (segment (start 36.25099 95.32101) (end 36.25099 98.989771) (width 0.25) (layer B.Cu) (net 43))
 (segment (start 38.1 93.472) (end 36.25099 95.32101) (width 0.25) (layer B.Cu) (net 43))
 (segment (start 46.363408 93.472) (end 32.081418 107.75399) (width 0.25) (layer B.Cu) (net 43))
 (segment (start 50.6 93.472) (end 46.363408 93.472) (width 0.25) (layer B.Cu) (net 43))
 (segment (start 38.1 78.232) (end 37.074999 77.206999) (width 0.25) (layer B.Cu) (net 1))
 (segment (start 38.1 78.232) (end 28.448 78.232) (width 0.25) (layer B.Cu) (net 1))
 (segment (start 50.6 78.232) (end 60.584 78.232) (width 0.25) (layer B.Cu) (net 1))
 (segment (start 38.1 78.232) (end 50.6 78.232) (width 0.25) (layer B.Cu) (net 1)))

